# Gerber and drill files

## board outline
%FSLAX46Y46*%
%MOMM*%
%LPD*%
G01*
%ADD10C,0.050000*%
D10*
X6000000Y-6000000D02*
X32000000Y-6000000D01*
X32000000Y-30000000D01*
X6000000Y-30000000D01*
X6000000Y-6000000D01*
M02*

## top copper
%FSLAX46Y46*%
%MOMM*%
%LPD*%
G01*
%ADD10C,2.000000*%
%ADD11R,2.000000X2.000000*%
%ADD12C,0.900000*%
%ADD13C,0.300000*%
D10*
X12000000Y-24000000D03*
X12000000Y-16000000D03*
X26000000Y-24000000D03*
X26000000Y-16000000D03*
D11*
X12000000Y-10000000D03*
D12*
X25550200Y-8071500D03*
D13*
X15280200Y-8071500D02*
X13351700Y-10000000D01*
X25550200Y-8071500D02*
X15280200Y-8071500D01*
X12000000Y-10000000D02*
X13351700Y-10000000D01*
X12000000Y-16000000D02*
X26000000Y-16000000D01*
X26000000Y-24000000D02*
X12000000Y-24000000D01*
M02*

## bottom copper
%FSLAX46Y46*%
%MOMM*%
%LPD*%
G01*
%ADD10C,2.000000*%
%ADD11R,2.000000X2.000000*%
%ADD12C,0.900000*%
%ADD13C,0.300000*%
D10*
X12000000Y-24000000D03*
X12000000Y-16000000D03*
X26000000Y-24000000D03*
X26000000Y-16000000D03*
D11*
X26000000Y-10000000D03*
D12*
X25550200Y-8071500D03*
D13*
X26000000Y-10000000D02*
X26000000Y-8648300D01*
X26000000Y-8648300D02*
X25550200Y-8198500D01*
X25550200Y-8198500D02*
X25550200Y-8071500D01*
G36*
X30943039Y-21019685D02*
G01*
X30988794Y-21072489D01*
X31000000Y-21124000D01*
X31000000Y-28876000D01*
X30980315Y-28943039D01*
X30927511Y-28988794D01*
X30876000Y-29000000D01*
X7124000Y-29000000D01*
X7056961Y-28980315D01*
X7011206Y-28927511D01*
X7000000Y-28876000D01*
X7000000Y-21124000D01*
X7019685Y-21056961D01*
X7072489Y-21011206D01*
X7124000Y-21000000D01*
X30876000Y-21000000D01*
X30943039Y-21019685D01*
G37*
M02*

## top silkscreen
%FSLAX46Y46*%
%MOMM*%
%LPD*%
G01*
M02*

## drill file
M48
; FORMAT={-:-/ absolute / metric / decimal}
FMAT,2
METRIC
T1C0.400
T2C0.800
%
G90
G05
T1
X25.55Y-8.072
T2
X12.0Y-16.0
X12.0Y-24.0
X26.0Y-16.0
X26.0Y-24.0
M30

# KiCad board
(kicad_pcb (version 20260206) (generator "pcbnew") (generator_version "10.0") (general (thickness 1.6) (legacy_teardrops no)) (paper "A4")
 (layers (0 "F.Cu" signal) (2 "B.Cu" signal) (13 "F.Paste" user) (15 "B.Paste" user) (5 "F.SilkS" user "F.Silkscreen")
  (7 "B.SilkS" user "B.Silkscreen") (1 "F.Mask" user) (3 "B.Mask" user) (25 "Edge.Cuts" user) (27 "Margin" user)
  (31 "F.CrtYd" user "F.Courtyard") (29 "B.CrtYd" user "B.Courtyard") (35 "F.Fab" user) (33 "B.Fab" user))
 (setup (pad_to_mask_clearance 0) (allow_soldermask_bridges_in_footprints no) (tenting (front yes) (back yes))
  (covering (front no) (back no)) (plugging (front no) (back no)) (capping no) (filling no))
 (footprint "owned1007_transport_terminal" (layer "F.Cu") (at 12 24)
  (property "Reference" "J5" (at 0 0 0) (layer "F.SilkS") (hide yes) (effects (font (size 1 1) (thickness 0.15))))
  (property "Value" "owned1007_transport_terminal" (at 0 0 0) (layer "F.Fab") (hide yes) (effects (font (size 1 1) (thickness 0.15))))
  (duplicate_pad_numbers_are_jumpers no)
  (pad "1" thru_hole circle (at 0 0) (size 2 2) (drill 0.8) (layers "*.Cu" "*.Mask") (remove_unused_layers no) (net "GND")))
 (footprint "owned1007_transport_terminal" (layer "F.Cu") (at 12 16)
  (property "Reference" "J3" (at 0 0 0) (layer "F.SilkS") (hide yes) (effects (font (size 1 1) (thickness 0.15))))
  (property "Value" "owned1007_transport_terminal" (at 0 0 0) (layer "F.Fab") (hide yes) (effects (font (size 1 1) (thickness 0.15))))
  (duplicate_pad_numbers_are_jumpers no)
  (pad "1" thru_hole circle (at 0 0) (size 2 2) (drill 0.8) (layers "*.Cu" "*.Mask") (remove_unused_layers no) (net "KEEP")))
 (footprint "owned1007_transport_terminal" (layer "F.Cu") (at 26 24)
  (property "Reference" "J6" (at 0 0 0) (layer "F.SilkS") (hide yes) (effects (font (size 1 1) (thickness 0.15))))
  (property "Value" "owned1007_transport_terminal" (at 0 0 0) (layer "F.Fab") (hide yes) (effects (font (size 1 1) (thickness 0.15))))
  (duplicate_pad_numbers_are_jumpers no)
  (pad "1" thru_hole circle (at 0 0) (size 2 2) (drill 0.8) (layers "*.Cu" "*.Mask") (remove_unused_layers no) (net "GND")))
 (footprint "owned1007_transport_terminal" (layer "F.Cu") (at 26 16)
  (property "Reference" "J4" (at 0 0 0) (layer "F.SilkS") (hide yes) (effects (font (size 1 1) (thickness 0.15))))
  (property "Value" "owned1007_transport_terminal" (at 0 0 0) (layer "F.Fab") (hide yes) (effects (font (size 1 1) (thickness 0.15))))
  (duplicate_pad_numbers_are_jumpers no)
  (pad "1" thru_hole circle (at 0 0) (size 2 2) (drill 0.8) (layers "*.Cu" "*.Mask") (remove_unused_layers no) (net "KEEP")))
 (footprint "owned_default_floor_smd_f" (layer "F.Cu") (at 12 10)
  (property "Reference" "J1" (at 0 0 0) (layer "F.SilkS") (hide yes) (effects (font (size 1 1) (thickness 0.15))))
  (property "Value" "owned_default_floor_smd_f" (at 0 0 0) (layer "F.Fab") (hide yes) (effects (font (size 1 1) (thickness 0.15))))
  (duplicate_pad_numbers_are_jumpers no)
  (pad "1" smd rect (at 0 0) (size 2 2) (layers "F.Cu" "F.Mask" "F.Paste") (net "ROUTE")))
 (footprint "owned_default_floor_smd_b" (layer "B.Cu") (at 26 10)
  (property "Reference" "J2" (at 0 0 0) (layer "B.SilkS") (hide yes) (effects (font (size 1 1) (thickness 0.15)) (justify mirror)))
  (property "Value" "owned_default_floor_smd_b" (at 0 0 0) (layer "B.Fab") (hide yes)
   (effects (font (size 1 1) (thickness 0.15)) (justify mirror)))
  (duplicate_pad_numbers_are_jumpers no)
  (pad "1" smd rect (at 0 0) (size 2 2) (layers "B.Cu" "B.Mask" "B.Paste") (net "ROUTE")))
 (gr_rect (start 6 6) (end 32 30) (stroke (width 0.05) (type default)) (fill no) (layer "Edge.Cuts"))
 (segment (start 15.2802 8.0715) (end 13.3517 10) (width 0.3) (layer "F.Cu") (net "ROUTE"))
 (segment (start 25.5502 8.0715) (end 15.2802 8.0715) (width 0.3) (layer "F.Cu") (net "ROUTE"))
 (segment (start 12 10) (end 13.3517 10) (width 0.3) (layer "F.Cu") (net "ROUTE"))
 (via (at 25.5502 8.0715) (size 0.9) (drill 0.4) (layers "F.Cu" "B.Cu") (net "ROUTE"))
 (segment (start 26 10) (end 26 8.6483) (width 0.3) (layer "B.Cu") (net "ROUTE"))
 (segment (start 26 8.6483) (end 25.5502 8.1985) (width 0.3) (layer "B.Cu") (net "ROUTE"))
 (segment (start 25.5502 8.1985) (end 25.5502 8.0715) (width 0.3) (layer "B.Cu") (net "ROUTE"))
 (segment (start 12 16) (end 26 16) (width 0.3) (locked yes) (layer "F.Cu") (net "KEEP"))
 (segment (start 26 24) (end 12 24) (width 0.3) (layer "F.Cu") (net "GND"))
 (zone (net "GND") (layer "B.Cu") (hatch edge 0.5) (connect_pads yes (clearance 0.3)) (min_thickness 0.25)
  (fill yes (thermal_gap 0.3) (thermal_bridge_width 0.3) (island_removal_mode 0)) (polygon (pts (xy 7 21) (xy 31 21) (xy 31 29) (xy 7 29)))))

